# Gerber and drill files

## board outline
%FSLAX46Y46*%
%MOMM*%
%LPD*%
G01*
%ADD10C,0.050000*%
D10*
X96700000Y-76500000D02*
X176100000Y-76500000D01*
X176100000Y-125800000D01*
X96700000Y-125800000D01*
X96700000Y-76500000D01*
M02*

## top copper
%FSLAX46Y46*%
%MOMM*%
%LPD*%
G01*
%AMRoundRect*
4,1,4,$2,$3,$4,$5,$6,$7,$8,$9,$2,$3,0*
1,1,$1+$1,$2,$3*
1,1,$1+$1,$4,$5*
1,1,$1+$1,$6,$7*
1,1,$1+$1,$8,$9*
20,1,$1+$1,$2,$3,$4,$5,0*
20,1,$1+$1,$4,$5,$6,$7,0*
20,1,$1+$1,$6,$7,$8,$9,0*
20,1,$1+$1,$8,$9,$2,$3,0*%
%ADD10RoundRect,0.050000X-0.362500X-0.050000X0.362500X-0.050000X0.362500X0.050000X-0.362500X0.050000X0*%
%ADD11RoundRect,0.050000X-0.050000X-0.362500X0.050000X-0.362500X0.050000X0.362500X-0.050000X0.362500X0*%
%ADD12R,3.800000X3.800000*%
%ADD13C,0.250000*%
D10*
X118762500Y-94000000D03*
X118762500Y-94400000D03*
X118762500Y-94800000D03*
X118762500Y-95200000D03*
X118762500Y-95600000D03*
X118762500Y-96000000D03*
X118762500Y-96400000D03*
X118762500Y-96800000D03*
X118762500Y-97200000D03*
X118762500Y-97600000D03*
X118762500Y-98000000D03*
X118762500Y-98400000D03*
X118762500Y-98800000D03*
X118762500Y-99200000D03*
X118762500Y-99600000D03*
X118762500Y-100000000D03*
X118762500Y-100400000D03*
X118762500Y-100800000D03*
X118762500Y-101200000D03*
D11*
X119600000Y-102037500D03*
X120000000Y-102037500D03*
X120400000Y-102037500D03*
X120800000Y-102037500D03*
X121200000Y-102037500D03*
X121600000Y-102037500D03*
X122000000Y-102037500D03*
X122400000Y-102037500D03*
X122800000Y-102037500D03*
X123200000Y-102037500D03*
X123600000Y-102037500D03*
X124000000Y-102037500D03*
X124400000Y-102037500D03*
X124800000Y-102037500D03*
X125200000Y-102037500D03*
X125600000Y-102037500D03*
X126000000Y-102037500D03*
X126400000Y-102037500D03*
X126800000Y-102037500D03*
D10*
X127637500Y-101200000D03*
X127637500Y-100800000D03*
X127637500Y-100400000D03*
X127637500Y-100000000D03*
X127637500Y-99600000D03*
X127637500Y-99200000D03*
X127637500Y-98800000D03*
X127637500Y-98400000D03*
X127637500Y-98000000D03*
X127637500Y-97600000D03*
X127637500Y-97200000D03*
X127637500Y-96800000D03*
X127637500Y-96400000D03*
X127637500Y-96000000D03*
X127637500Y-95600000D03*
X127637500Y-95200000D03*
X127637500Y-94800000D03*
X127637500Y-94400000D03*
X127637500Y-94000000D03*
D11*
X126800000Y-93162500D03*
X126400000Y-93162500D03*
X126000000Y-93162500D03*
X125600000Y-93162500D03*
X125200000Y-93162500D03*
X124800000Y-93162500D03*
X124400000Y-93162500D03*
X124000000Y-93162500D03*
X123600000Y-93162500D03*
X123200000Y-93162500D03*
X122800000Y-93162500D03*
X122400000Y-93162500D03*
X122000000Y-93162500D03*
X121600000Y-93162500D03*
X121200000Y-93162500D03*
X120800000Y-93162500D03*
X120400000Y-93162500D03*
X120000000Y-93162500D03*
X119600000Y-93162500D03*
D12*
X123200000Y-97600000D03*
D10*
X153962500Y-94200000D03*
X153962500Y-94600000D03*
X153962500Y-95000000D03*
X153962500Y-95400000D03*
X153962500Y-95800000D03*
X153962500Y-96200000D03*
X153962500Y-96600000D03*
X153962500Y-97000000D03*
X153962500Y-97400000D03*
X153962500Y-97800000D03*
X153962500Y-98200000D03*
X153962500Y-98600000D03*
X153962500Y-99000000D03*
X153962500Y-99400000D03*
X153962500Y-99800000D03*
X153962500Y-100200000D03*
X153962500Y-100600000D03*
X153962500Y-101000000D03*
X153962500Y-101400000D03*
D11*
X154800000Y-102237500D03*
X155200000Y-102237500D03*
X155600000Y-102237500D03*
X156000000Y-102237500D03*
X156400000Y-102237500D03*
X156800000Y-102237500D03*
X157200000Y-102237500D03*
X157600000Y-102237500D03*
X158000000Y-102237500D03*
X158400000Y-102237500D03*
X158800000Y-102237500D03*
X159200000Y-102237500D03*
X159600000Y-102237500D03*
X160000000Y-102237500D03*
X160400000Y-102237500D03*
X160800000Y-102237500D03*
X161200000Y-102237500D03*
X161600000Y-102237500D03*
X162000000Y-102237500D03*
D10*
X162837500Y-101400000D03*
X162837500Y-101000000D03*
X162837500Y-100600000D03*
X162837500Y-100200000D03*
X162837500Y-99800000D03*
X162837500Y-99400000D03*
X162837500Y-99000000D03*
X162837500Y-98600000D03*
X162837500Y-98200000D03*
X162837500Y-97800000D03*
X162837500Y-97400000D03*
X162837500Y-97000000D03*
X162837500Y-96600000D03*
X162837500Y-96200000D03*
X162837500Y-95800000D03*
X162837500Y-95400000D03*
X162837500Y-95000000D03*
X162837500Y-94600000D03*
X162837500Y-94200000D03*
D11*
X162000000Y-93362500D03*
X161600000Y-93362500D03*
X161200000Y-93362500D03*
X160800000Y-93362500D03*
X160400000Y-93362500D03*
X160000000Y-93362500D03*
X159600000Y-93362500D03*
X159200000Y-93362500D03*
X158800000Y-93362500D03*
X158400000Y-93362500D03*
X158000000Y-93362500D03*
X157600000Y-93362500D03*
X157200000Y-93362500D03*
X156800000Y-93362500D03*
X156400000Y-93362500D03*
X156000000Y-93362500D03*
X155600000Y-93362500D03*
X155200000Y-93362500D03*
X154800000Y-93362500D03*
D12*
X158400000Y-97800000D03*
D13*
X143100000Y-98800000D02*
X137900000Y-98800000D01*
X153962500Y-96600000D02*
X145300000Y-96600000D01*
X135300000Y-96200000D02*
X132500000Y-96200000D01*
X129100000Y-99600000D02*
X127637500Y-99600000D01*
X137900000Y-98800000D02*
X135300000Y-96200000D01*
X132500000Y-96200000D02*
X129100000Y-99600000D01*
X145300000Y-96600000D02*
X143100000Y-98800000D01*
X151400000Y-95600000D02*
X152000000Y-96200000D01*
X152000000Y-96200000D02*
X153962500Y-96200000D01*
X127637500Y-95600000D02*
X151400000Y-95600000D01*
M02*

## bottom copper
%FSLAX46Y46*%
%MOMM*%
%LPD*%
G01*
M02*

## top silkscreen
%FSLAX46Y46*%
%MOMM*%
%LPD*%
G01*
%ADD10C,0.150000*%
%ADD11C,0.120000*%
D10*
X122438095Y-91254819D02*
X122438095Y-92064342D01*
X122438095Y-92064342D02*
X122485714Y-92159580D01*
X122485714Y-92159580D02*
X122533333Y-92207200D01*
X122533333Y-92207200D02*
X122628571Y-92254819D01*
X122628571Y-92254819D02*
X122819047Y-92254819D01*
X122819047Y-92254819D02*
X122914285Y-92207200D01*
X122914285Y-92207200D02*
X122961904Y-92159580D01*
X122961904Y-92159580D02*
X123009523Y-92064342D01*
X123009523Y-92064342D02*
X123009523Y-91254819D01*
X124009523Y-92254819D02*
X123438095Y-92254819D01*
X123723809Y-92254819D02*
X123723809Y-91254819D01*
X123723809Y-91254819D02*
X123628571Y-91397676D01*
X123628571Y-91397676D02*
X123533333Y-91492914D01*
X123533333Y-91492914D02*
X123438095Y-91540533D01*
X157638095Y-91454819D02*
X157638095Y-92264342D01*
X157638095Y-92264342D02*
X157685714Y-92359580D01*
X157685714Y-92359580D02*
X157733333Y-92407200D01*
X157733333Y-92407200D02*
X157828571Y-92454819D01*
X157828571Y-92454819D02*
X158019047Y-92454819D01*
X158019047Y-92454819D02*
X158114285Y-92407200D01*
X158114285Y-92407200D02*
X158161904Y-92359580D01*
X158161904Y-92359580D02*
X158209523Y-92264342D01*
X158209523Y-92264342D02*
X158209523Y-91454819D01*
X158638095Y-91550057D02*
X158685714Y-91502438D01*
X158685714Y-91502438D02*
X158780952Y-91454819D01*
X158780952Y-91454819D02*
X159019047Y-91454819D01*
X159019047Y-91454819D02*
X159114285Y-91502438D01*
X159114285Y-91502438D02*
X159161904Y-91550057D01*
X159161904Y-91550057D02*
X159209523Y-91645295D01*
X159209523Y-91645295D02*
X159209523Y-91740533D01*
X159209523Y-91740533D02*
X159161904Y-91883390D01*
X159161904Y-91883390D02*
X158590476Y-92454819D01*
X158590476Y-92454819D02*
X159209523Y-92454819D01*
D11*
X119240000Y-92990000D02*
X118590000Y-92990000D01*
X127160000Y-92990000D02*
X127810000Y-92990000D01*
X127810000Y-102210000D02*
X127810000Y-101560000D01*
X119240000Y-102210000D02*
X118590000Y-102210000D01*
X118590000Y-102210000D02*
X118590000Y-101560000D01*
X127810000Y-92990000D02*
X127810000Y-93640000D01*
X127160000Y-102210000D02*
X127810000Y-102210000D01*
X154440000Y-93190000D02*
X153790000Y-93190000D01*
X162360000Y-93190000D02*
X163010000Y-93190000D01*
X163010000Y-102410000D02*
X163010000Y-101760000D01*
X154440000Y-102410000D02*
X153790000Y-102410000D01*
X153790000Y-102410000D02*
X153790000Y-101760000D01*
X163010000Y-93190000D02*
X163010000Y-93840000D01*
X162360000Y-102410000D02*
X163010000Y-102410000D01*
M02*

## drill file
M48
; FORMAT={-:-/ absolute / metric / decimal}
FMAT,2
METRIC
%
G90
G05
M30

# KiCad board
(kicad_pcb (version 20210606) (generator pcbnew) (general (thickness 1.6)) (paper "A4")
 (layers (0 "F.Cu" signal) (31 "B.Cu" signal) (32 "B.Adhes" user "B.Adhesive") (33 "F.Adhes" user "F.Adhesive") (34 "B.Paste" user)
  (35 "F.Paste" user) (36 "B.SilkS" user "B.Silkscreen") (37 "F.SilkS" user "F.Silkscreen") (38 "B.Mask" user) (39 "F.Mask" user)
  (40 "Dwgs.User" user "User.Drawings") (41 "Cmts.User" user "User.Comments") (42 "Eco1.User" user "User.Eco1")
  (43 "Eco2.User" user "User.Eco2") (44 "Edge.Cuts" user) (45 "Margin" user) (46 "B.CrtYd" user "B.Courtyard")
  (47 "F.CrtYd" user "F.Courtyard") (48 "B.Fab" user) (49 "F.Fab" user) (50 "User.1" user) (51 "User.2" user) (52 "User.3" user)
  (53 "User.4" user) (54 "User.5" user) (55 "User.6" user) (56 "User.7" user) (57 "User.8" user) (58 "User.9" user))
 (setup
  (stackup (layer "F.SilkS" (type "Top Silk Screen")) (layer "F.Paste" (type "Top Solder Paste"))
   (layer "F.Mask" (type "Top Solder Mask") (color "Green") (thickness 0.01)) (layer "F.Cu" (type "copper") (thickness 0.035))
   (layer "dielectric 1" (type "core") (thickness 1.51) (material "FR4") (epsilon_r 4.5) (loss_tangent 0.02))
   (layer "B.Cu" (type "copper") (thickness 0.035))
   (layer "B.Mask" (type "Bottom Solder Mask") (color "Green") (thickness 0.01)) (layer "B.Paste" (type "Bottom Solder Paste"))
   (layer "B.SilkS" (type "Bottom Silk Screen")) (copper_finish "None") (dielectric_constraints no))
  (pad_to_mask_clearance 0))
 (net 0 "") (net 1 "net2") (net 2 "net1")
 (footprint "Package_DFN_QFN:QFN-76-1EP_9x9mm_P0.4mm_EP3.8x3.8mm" (layer "F.Cu") (at 123.2 97.6)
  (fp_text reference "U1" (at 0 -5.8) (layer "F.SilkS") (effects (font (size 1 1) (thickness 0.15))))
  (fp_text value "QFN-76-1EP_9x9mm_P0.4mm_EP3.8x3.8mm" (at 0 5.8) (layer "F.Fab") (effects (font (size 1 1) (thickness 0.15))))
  (fp_line (start -3.96 -4.61) (end -4.61 -4.61) (layer "F.SilkS") (width 0.12))
  (fp_line (start 3.96 -4.61) (end 4.61 -4.61) (layer "F.SilkS") (width 0.12))
  (fp_line (start 4.61 4.61) (end 4.61 3.96) (layer "F.SilkS") (width 0.12))
  (fp_line (start -3.96 4.61) (end -4.61 4.61) (layer "F.SilkS") (width 0.12))
  (fp_line (start -4.61 4.61) (end -4.61 3.96) (layer "F.SilkS") (width 0.12))
  (fp_line (start 4.61 -4.61) (end 4.61 -3.96) (layer "F.SilkS") (width 0.12))
  (fp_line (start 3.96 4.61) (end 4.61 4.61) (layer "F.SilkS") (width 0.12))
  (pad "" smd roundrect locked (at 0 -1.27) (size 1.02 1.02) (layers "F.Paste") (roundrect_rratio 0.245098))
  (pad "" smd roundrect locked (at 1.27 -1.27) (size 1.02 1.02) (layers "F.Paste") (roundrect_rratio 0.245098))
  (pad "" smd roundrect locked (at -1.27 -1.27) (size 1.02 1.02) (layers "F.Paste") (roundrect_rratio 0.245098))
  (pad "" smd roundrect locked (at 1.27 1.27) (size 1.02 1.02) (layers "F.Paste") (roundrect_rratio 0.245098))
  (pad "" smd roundrect locked (at 1.27 0) (size 1.02 1.02) (layers "F.Paste") (roundrect_rratio 0.245098))
  (pad "" smd roundrect locked (at -1.27 1.27) (size 1.02 1.02) (layers "F.Paste") (roundrect_rratio 0.245098))
  (pad "" smd roundrect locked (at 0 1.27) (size 1.02 1.02) (layers "F.Paste") (roundrect_rratio 0.245098))
  (pad "" smd roundrect locked (at 0 0) (size 1.02 1.02) (layers "F.Paste") (roundrect_rratio 0.245098))
  (pad "" smd roundrect locked (at -1.27 0) (size 1.02 1.02) (layers "F.Paste") (roundrect_rratio 0.245098))
  (pad "1" smd roundrect locked (at -4.4375 -3.6) (size 0.825 0.2) (layers "F.Cu" "F.Paste" "F.Mask") (roundrect_rratio 0.25))
  (pad "2" smd roundrect locked (at -4.4375 -3.2) (size 0.825 0.2) (layers "F.Cu" "F.Paste" "F.Mask") (roundrect_rratio 0.25))
  (pad "3" smd roundrect locked (at -4.4375 -2.8) (size 0.825 0.2) (layers "F.Cu" "F.Paste" "F.Mask") (roundrect_rratio 0.25))
  (pad "4" smd roundrect locked (at -4.4375 -2.4) (size 0.825 0.2) (layers "F.Cu" "F.Paste" "F.Mask") (roundrect_rratio 0.25))
  (pad "5" smd roundrect locked (at -4.4375 -2) (size 0.825 0.2) (layers "F.Cu" "F.Paste" "F.Mask") (roundrect_rratio 0.25))
  (pad "6" smd roundrect locked (at -4.4375 -1.6) (size 0.825 0.2) (layers "F.Cu" "F.Paste" "F.Mask") (roundrect_rratio 0.25))
  (pad "7" smd roundrect locked (at -4.4375 -1.2) (size 0.825 0.2) (layers "F.Cu" "F.Paste" "F.Mask") (roundrect_rratio 0.25))
  (pad "8" smd roundrect locked (at -4.4375 -0.8) (size 0.825 0.2) (layers "F.Cu" "F.Paste" "F.Mask") (roundrect_rratio 0.25))
  (pad "9" smd roundrect locked (at -4.4375 -0.4) (size 0.825 0.2) (layers "F.Cu" "F.Paste" "F.Mask") (roundrect_rratio 0.25))
  (pad "10" smd roundrect locked (at -4.4375 0) (size 0.825 0.2) (layers "F.Cu" "F.Paste" "F.Mask") (roundrect_rratio 0.25))
  (pad "11" smd roundrect locked (at -4.4375 0.4) (size 0.825 0.2) (layers "F.Cu" "F.Paste" "F.Mask") (roundrect_rratio 0.25))
  (pad "12" smd roundrect locked (at -4.4375 0.8) (size 0.825 0.2) (layers "F.Cu" "F.Paste" "F.Mask") (roundrect_rratio 0.25))
  (pad "13" smd roundrect locked (at -4.4375 1.2) (size 0.825 0.2) (layers "F.Cu" "F.Paste" "F.Mask") (roundrect_rratio 0.25))
  (pad "14" smd roundrect locked (at -4.4375 1.6) (size 0.825 0.2) (layers "F.Cu" "F.Paste" "F.Mask") (roundrect_rratio 0.25))
  (pad "15" smd roundrect locked (at -4.4375 2) (size 0.825 0.2) (layers "F.Cu" "F.Paste" "F.Mask") (roundrect_rratio 0.25))
  (pad "16" smd roundrect locked (at -4.4375 2.4) (size 0.825 0.2) (layers "F.Cu" "F.Paste" "F.Mask") (roundrect_rratio 0.25))
  (pad "17" smd roundrect locked (at -4.4375 2.8) (size 0.825 0.2) (layers "F.Cu" "F.Paste" "F.Mask") (roundrect_rratio 0.25))
  (pad "18" smd roundrect locked (at -4.4375 3.2) (size 0.825 0.2) (layers "F.Cu" "F.Paste" "F.Mask") (roundrect_rratio 0.25))
  (pad "19" smd roundrect locked (at -4.4375 3.6) (size 0.825 0.2) (layers "F.Cu" "F.Paste" "F.Mask") (roundrect_rratio 0.25))
  (pad "20" smd roundrect locked (at -3.6 4.4375) (size 0.2 0.825) (layers "F.Cu" "F.Paste" "F.Mask") (roundrect_rratio 0.25))
  (pad "21" smd roundrect locked (at -3.2 4.4375) (size 0.2 0.825) (layers "F.Cu" "F.Paste" "F.Mask") (roundrect_rratio 0.25))
  (pad "22" smd roundrect locked (at -2.8 4.4375) (size 0.2 0.825) (layers "F.Cu" "F.Paste" "F.Mask") (roundrect_rratio 0.25))
  (pad "23" smd roundrect locked (at -2.4 4.4375) (size 0.2 0.825) (layers "F.Cu" "F.Paste" "F.Mask") (roundrect_rratio 0.25))
  (pad "24" smd roundrect locked (at -2 4.4375) (size 0.2 0.825) (layers "F.Cu" "F.Paste" "F.Mask") (roundrect_rratio 0.25))
  (pad "25" smd roundrect locked (at -1.6 4.4375) (size 0.2 0.825) (layers "F.Cu" "F.Paste" "F.Mask") (roundrect_rratio 0.25))
  (pad "26" smd roundrect locked (at -1.2 4.4375) (size 0.2 0.825) (layers "F.Cu" "F.Paste" "F.Mask") (roundrect_rratio 0.25))
  (pad "27" smd roundrect locked (at -0.8 4.4375) (size 0.2 0.825) (layers "F.Cu" "F.Paste" "F.Mask") (roundrect_rratio 0.25))
  (pad "28" smd roundrect locked (at -0.4 4.4375) (size 0.2 0.825) (layers "F.Cu" "F.Paste" "F.Mask") (roundrect_rratio 0.25))
  (pad "29" smd roundrect locked (at 0 4.4375) (size 0.2 0.825) (layers "F.Cu" "F.Paste" "F.Mask") (roundrect_rratio 0.25))
  (pad "30" smd roundrect locked (at 0.4 4.4375) (size 0.2 0.825) (layers "F.Cu" "F.Paste" "F.Mask") (roundrect_rratio 0.25))
  (pad "31" smd roundrect locked (at 0.8 4.4375) (size 0.2 0.825) (layers "F.Cu" "F.Paste" "F.Mask") (roundrect_rratio 0.25))
  (pad "32" smd roundrect locked (at 1.2 4.4375) (size 0.2 0.825) (layers "F.Cu" "F.Paste" "F.Mask") (roundrect_rratio 0.25))
  (pad "33" smd roundrect locked (at 1.6 4.4375) (size 0.2 0.825) (layers "F.Cu" "F.Paste" "F.Mask") (roundrect_rratio 0.25))
  (pad "34" smd roundrect locked (at 2 4.4375) (size 0.2 0.825) (layers "F.Cu" "F.Paste" "F.Mask") (roundrect_rratio 0.25))
  (pad "35" smd roundrect locked (at 2.4 4.4375) (size 0.2 0.825) (layers "F.Cu" "F.Paste" "F.Mask") (roundrect_rratio 0.25))
  (pad "36" smd roundrect locked (at 2.8 4.4375) (size 0.2 0.825) (layers "F.Cu" "F.Paste" "F.Mask") (roundrect_rratio 0.25))
  (pad "37" smd roundrect locked (at 3.2 4.4375) (size 0.2 0.825) (layers "F.Cu" "F.Paste" "F.Mask") (roundrect_rratio 0.25))
  (pad "38" smd roundrect locked (at 3.6 4.4375) (size 0.2 0.825) (layers "F.Cu" "F.Paste" "F.Mask") (roundrect_rratio 0.25))
  (pad "39" smd roundrect locked (at 4.4375 3.6) (size 0.825 0.2) (layers "F.Cu" "F.Paste" "F.Mask") (roundrect_rratio 0.25))
  (pad "40" smd roundrect locked (at 4.4375 3.2) (size 0.825 0.2) (layers "F.Cu" "F.Paste" "F.Mask") (roundrect_rratio 0.25))
  (pad "41" smd roundrect locked (at 4.4375 2.8) (size 0.825 0.2) (layers "F.Cu" "F.Paste" "F.Mask") (roundrect_rratio 0.25))
  (pad "42" smd roundrect locked (at 4.4375 2.4) (size 0.825 0.2) (layers "F.Cu" "F.Paste" "F.Mask") (roundrect_rratio 0.25))
  (pad "43" smd roundrect locked (at 4.4375 2) (size 0.825 0.2) (layers "F.Cu" "F.Paste" "F.Mask") (roundrect_rratio 0.25) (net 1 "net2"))
  (pad "44" smd roundrect locked (at 4.4375 1.6) (size 0.825 0.2) (layers "F.Cu" "F.Paste" "F.Mask") (roundrect_rratio 0.25))
  (pad "45" smd roundrect locked (at 4.4375 1.2) (size 0.825 0.2) (layers "F.Cu" "F.Paste" "F.Mask") (roundrect_rratio 0.25))
  (pad "46" smd roundrect locked (at 4.4375 0.8) (size 0.825 0.2) (layers "F.Cu" "F.Paste" "F.Mask") (roundrect_rratio 0.25))
  (pad "47" smd roundrect locked (at 4.4375 0.4) (size 0.825 0.2) (layers "F.Cu" "F.Paste" "F.Mask") (roundrect_rratio 0.25))
  (pad "48" smd roundrect locked (at 4.4375 0) (size 0.825 0.2) (layers "F.Cu" "F.Paste" "F.Mask") (roundrect_rratio 0.25))
  (pad "49" smd roundrect locked (at 4.4375 -0.4) (size 0.825 0.2) (layers "F.Cu" "F.Paste" "F.Mask") (roundrect_rratio 0.25))
  (pad "50" smd roundrect locked (at 4.4375 -0.8) (size 0.825 0.2) (layers "F.Cu" "F.Paste" "F.Mask") (roundrect_rratio 0.25))
  (pad "51" smd roundrect locked (at 4.4375 -1.2) (size 0.825 0.2) (layers "F.Cu" "F.Paste" "F.Mask") (roundrect_rratio 0.25))
  (pad "52" smd roundrect locked (at 4.4375 -1.6) (size 0.825 0.2) (layers "F.Cu" "F.Paste" "F.Mask") (roundrect_rratio 0.25))
  (pad "53" smd roundrect locked (at 4.4375 -2) (size 0.825 0.2) (layers "F.Cu" "F.Paste" "F.Mask") (roundrect_rratio 0.25) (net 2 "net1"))
  (pad "54" smd roundrect locked (at 4.4375 -2.4) (size 0.825 0.2) (layers "F.Cu" "F.Paste" "F.Mask") (roundrect_rratio 0.25))
  (pad "55" smd roundrect locked (at 4.4375 -2.8) (size 0.825 0.2) (layers "F.Cu" "F.Paste" "F.Mask") (roundrect_rratio 0.25))
  (pad "56" smd roundrect locked (at 4.4375 -3.2) (size 0.825 0.2) (layers "F.Cu" "F.Paste" "F.Mask") (roundrect_rratio 0.25))
  (pad "57" smd roundrect locked (at 4.4375 -3.6) (size 0.825 0.2) (layers "F.Cu" "F.Paste" "F.Mask") (roundrect_rratio 0.25))
  (pad "58" smd roundrect locked (at 3.6 -4.4375) (size 0.2 0.825) (layers "F.Cu" "F.Paste" "F.Mask") (roundrect_rratio 0.25))
  (pad "59" smd roundrect locked (at 3.2 -4.4375) (size 0.2 0.825) (layers "F.Cu" "F.Paste" "F.Mask") (roundrect_rratio 0.25))
  (pad "60" smd roundrect locked (at 2.8 -4.4375) (size 0.2 0.825) (layers "F.Cu" "F.Paste" "F.Mask") (roundrect_rratio 0.25))
  (pad "61" smd roundrect locked (at 2.4 -4.4375) (size 0.2 0.825) (layers "F.Cu" "F.Paste" "F.Mask") (roundrect_rratio 0.25))
  (pad "62" smd roundrect locked (at 2 -4.4375) (size 0.2 0.825) (layers "F.Cu" "F.Paste" "F.Mask") (roundrect_rratio 0.25))
  (pad "63" smd roundrect locked (at 1.6 -4.4375) (size 0.2 0.825) (layers "F.Cu" "F.Paste" "F.Mask") (roundrect_rratio 0.25))
  (pad "64" smd roundrect locked (at 1.2 -4.4375) (size 0.2 0.825) (layers "F.Cu" "F.Paste" "F.Mask") (roundrect_rratio 0.25))
  (pad "65" smd roundrect locked (at 0.8 -4.4375) (size 0.2 0.825) (layers "F.Cu" "F.Paste" "F.Mask") (roundrect_rratio 0.25))
  (pad "66" smd roundrect locked (at 0.4 -4.4375) (size 0.2 0.825) (layers "F.Cu" "F.Paste" "F.Mask") (roundrect_rratio 0.25))
  (pad "67" smd roundrect locked (at 0 -4.4375) (size 0.2 0.825) (layers "F.Cu" "F.Paste" "F.Mask") (roundrect_rratio 0.25))
  (pad "68" smd roundrect locked (at -0.4 -4.4375) (size 0.2 0.825) (layers "F.Cu" "F.Paste" "F.Mask") (roundrect_rratio 0.25))
  (pad "69" smd roundrect locked (at -0.8 -4.4375) (size 0.2 0.825) (layers "F.Cu" "F.Paste" "F.Mask") (roundrect_rratio 0.25))
  (pad "70" smd roundrect locked (at -1.2 -4.4375) (size 0.2 0.825) (layers "F.Cu" "F.Paste" "F.Mask") (roundrect_rratio 0.25))
  (pad "71" smd roundrect locked (at -1.6 -4.4375) (size 0.2 0.825) (layers "F.Cu" "F.Paste" "F.Mask") (roundrect_rratio 0.25))
  (pad "72" smd roundrect locked (at -2 -4.4375) (size 0.2 0.825) (layers "F.Cu" "F.Paste" "F.Mask") (roundrect_rratio 0.25))
  (pad "73" smd roundrect locked (at -2.4 -4.4375) (size 0.2 0.825) (layers "F.Cu" "F.Paste" "F.Mask") (roundrect_rratio 0.25))
  (pad "74" smd roundrect locked (at -2.8 -4.4375) (size 0.2 0.825) (layers "F.Cu" "F.Paste" "F.Mask") (roundrect_rratio 0.25))
  (pad "75" smd roundrect locked (at -3.2 -4.4375) (size 0.2 0.825) (layers "F.Cu" "F.Paste" "F.Mask") (roundrect_rratio 0.25))
  (pad "76" smd roundrect locked (at -3.6 -4.4375) (size 0.2 0.825) (layers "F.Cu" "F.Paste" "F.Mask") (roundrect_rratio 0.25))
  (pad "77" smd rect locked (at 0 0) (size 3.8 3.8) (layers "F.Cu" "F.Mask")))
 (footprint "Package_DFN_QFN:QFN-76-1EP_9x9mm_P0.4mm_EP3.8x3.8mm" (layer "F.Cu") (at 158.4 97.8)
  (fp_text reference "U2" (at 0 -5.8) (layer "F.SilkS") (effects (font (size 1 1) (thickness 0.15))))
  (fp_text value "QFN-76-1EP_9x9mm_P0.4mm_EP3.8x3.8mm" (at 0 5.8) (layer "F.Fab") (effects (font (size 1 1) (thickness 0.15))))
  (fp_line (start -3.96 -4.61) (end -4.61 -4.61) (layer "F.SilkS") (width 0.12))
  (fp_line (start 3.96 -4.61) (end 4.61 -4.61) (layer "F.SilkS") (width 0.12))
  (fp_line (start 4.61 4.61) (end 4.61 3.96) (layer "F.SilkS") (width 0.12))
  (fp_line (start -3.96 4.61) (end -4.61 4.61) (layer "F.SilkS") (width 0.12))
  (fp_line (start -4.61 4.61) (end -4.61 3.96) (layer "F.SilkS") (width 0.12))
  (fp_line (start 4.61 -4.61) (end 4.61 -3.96) (layer "F.SilkS") (width 0.12))
  (fp_line (start 3.96 4.61) (end 4.61 4.61) (layer "F.SilkS") (width 0.12))
  (pad "" smd roundrect locked (at 0 -1.27) (size 1.02 1.02) (layers "F.Paste") (roundrect_rratio 0.245098))
  (pad "" smd roundrect locked (at 1.27 -1.27) (size 1.02 1.02) (layers "F.Paste") (roundrect_rratio 0.245098))
  (pad "" smd roundrect locked (at -1.27 -1.27) (size 1.02 1.02) (layers "F.Paste") (roundrect_rratio 0.245098))
  (pad "" smd roundrect locked (at 1.27 1.27) (size 1.02 1.02) (layers "F.Paste") (roundrect_rratio 0.245098))
  (pad "" smd roundrect locked (at 1.27 0) (size 1.02 1.02) (layers "F.Paste") (roundrect_rratio 0.245098))
  (pad "" smd roundrect locked (at -1.27 1.27) (size 1.02 1.02) (layers "F.Paste") (roundrect_rratio 0.245098))
  (pad "" smd roundrect locked (at 0 1.27) (size 1.02 1.02) (layers "F.Paste") (roundrect_rratio 0.245098))
  (pad "" smd roundrect locked (at 0 0) (size 1.02 1.02) (layers "F.Paste") (roundrect_rratio 0.245098))
  (pad "" smd roundrect locked (at -1.27 0) (size 1.02 1.02) (layers "F.Paste") (roundrect_rratio 0.245098))
  (pad "1" smd roundrect locked (at -4.4375 -3.6) (size 0.825 0.2) (layers "F.Cu" "F.Paste" "F.Mask") (roundrect_rratio 0.25))
  (pad "2" smd roundrect locked (at -4.4375 -3.2) (size 0.825 0.2) (layers "F.Cu" "F.Paste" "F.Mask") (roundrect_rratio 0.25))
  (pad "3" smd roundrect locked (at -4.4375 -2.8) (size 0.825 0.2) (layers "F.Cu" "F.Paste" "F.Mask") (roundrect_rratio 0.25))
  (pad "4" smd roundrect locked (at -4.4375 -2.4) (size 0.825 0.2) (layers "F.Cu" "F.Paste" "F.Mask") (roundrect_rratio 0.25))
  (pad "5" smd roundrect locked (at -4.4375 -2) (size 0.825 0.2) (layers "F.Cu" "F.Paste" "F.Mask") (roundrect_rratio 0.25))
  (pad "6" smd roundrect locked (at -4.4375 -1.6) (size 0.825 0.2) (layers "F.Cu" "F.Paste" "F.Mask") (roundrect_rratio 0.25) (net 2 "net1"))
  (pad "7" smd roundrect locked (at -4.4375 -1.2) (size 0.825 0.2) (layers "F.Cu" "F.Paste" "F.Mask") (roundrect_rratio 0.25) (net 1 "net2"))
  (pad "8" smd roundrect locked (at -4.4375 -0.8) (size 0.825 0.2) (layers "F.Cu" "F.Paste" "F.Mask") (roundrect_rratio 0.25))
  (pad "9" smd roundrect locked (at -4.4375 -0.4) (size 0.825 0.2) (layers "F.Cu" "F.Paste" "F.Mask") (roundrect_rratio 0.25))
  (pad "10" smd roundrect locked (at -4.4375 0) (size 0.825 0.2) (layers "F.Cu" "F.Paste" "F.Mask") (roundrect_rratio 0.25))
  (pad "11" smd roundrect locked (at -4.4375 0.4) (size 0.825 0.2) (layers "F.Cu" "F.Paste" "F.Mask") (roundrect_rratio 0.25))
  (pad "12" smd roundrect locked (at -4.4375 0.8) (size 0.825 0.2) (layers "F.Cu" "F.Paste" "F.Mask") (roundrect_rratio 0.25))
  (pad "13" smd roundrect locked (at -4.4375 1.2) (size 0.825 0.2) (layers "F.Cu" "F.Paste" "F.Mask") (roundrect_rratio 0.25))
  (pad "14" smd roundrect locked (at -4.4375 1.6) (size 0.825 0.2) (layers "F.Cu" "F.Paste" "F.Mask") (roundrect_rratio 0.25))
  (pad "15" smd roundrect locked (at -4.4375 2) (size 0.825 0.2) (layers "F.Cu" "F.Paste" "F.Mask") (roundrect_rratio 0.25))
  (pad "16" smd roundrect locked (at -4.4375 2.4) (size 0.825 0.2) (layers "F.Cu" "F.Paste" "F.Mask") (roundrect_rratio 0.25))
  (pad "17" smd roundrect locked (at -4.4375 2.8) (size 0.825 0.2) (layers "F.Cu" "F.Paste" "F.Mask") (roundrect_rratio 0.25))
  (pad "18" smd roundrect locked (at -4.4375 3.2) (size 0.825 0.2) (layers "F.Cu" "F.Paste" "F.Mask") (roundrect_rratio 0.25))
  (pad "19" smd roundrect locked (at -4.4375 3.6) (size 0.825 0.2) (layers "F.Cu" "F.Paste" "F.Mask") (roundrect_rratio 0.25))
  (pad "20" smd roundrect locked (at -3.6 4.4375) (size 0.2 0.825) (layers "F.Cu" "F.Paste" "F.Mask") (roundrect_rratio 0.25))
  (pad "21" smd roundrect locked (at -3.2 4.4375) (size 0.2 0.825) (layers "F.Cu" "F.Paste" "F.Mask") (roundrect_rratio 0.25))
  (pad "22" smd roundrect locked (at -2.8 4.4375) (size 0.2 0.825) (layers "F.Cu" "F.Paste" "F.Mask") (roundrect_rratio 0.25))
  (pad "23" smd roundrect locked (at -2.4 4.4375) (size 0.2 0.825) (layers "F.Cu" "F.Paste" "F.Mask") (roundrect_rratio 0.25))
  (pad "24" smd roundrect locked (at -2 4.4375) (size 0.2 0.825) (layers "F.Cu" "F.Paste" "F.Mask") (roundrect_rratio 0.25))
  (pad "25" smd roundrect locked (at -1.6 4.4375) (size 0.2 0.825) (layers "F.Cu" "F.Paste" "F.Mask") (roundrect_rratio 0.25))
  (pad "26" smd roundrect locked (at -1.2 4.4375) (size 0.2 0.825) (layers "F.Cu" "F.Paste" "F.Mask") (roundrect_rratio 0.25))
  (pad "27" smd roundrect locked (at -0.8 4.4375) (size 0.2 0.825) (layers "F.Cu" "F.Paste" "F.Mask") (roundrect_rratio 0.25))
  (pad "28" smd roundrect locked (at -0.4 4.4375) (size 0.2 0.825) (layers "F.Cu" "F.Paste" "F.Mask") (roundrect_rratio 0.25))
  (pad "29" smd roundrect locked (at 0 4.4375) (size 0.2 0.825) (layers "F.Cu" "F.Paste" "F.Mask") (roundrect_rratio 0.25))
  (pad "30" smd roundrect locked (at 0.4 4.4375) (size 0.2 0.825) (layers "F.Cu" "F.Paste" "F.Mask") (roundrect_rratio 0.25))
  (pad "31" smd roundrect locked (at 0.8 4.4375) (size 0.2 0.825) (layers "F.Cu" "F.Paste" "F.Mask") (roundrect_rratio 0.25))
  (pad "32" smd roundrect locked (at 1.2 4.4375) (size 0.2 0.825) (layers "F.Cu" "F.Paste" "F.Mask") (roundrect_rratio 0.25))
  (pad "33" smd roundrect locked (at 1.6 4.4375) (size 0.2 0.825) (layers "F.Cu" "F.Paste" "F.Mask") (roundrect_rratio 0.25))
  (pad "34" smd roundrect locked (at 2 4.4375) (size 0.2 0.825) (layers "F.Cu" "F.Paste" "F.Mask") (roundrect_rratio 0.25))
  (pad "35" smd roundrect locked (at 2.4 4.4375) (size 0.2 0.825) (layers "F.Cu" "F.Paste" "F.Mask") (roundrect_rratio 0.25))
  (pad "36" smd roundrect locked (at 2.8 4.4375) (size 0.2 0.825) (layers "F.Cu" "F.Paste" "F.Mask") (roundrect_rratio 0.25))
  (pad "37" smd roundrect locked (at 3.2 4.4375) (size 0.2 0.825) (layers "F.Cu" "F.Paste" "F.Mask") (roundrect_rratio 0.25))
  (pad "38" smd roundrect locked (at 3.6 4.4375) (size 0.2 0.825) (layers "F.Cu" "F.Paste" "F.Mask") (roundrect_rratio 0.25))
  (pad "39" smd roundrect locked (at 4.4375 3.6) (size 0.825 0.2) (layers "F.Cu" "F.Paste" "F.Mask") (roundrect_rratio 0.25))
  (pad "40" smd roundrect locked (at 4.4375 3.2) (size 0.825 0.2) (layers "F.Cu" "F.Paste" "F.Mask") (roundrect_rratio 0.25))
  (pad "41" smd roundrect locked (at 4.4375 2.8) (size 0.825 0.2) (layers "F.Cu" "F.Paste" "F.Mask") (roundrect_rratio 0.25))
  (pad "42" smd roundrect locked (at 4.4375 2.4) (size 0.825 0.2) (layers "F.Cu" "F.Paste" "F.Mask") (roundrect_rratio 0.25))
  (pad "43" smd roundrect locked (at 4.4375 2) (size 0.825 0.2) (layers "F.Cu" "F.Paste" "F.Mask") (roundrect_rratio 0.25))
  (pad "44" smd roundrect locked (at 4.4375 1.6) (size 0.825 0.2) (layers "F.Cu" "F.Paste" "F.Mask") (roundrect_rratio 0.25))
  (pad "45" smd roundrect locked (at 4.4375 1.2) (size 0.825 0.2) (layers "F.Cu" "F.Paste" "F.Mask") (roundrect_rratio 0.25))
  (pad "46" smd roundrect locked (at 4.4375 0.8) (size 0.825 0.2) (layers "F.Cu" "F.Paste" "F.Mask") (roundrect_rratio 0.25))
  (pad "47" smd roundrect locked (at 4.4375 0.4) (size 0.825 0.2) (layers "F.Cu" "F.Paste" "F.Mask") (roundrect_rratio 0.25))
  (pad "48" smd roundrect locked (at 4.4375 0) (size 0.825 0.2) (layers "F.Cu" "F.Paste" "F.Mask") (roundrect_rratio 0.25))
  (pad "49" smd roundrect locked (at 4.4375 -0.4) (size 0.825 0.2) (layers "F.Cu" "F.Paste" "F.Mask") (roundrect_rratio 0.25))
  (pad "50" smd roundrect locked (at 4.4375 -0.8) (size 0.825 0.2) (layers "F.Cu" "F.Paste" "F.Mask") (roundrect_rratio 0.25))
  (pad "51" smd roundrect locked (at 4.4375 -1.2) (size 0.825 0.2) (layers "F.Cu" "F.Paste" "F.Mask") (roundrect_rratio 0.25))
  (pad "52" smd roundrect locked (at 4.4375 -1.6) (size 0.825 0.2) (layers "F.Cu" "F.Paste" "F.Mask") (roundrect_rratio 0.25))
  (pad "53" smd roundrect locked (at 4.4375 -2) (size 0.825 0.2) (layers "F.Cu" "F.Paste" "F.Mask") (roundrect_rratio 0.25))
  (pad "54" smd roundrect locked (at 4.4375 -2.4) (size 0.825 0.2) (layers "F.Cu" "F.Paste" "F.Mask") (roundrect_rratio 0.25))
  (pad "55" smd roundrect locked (at 4.4375 -2.8) (size 0.825 0.2) (layers "F.Cu" "F.Paste" "F.Mask") (roundrect_rratio 0.25))
  (pad "56" smd roundrect locked (at 4.4375 -3.2) (size 0.825 0.2) (layers "F.Cu" "F.Paste" "F.Mask") (roundrect_rratio 0.25))
  (pad "57" smd roundrect locked (at 4.4375 -3.6) (size 0.825 0.2) (layers "F.Cu" "F.Paste" "F.Mask") (roundrect_rratio 0.25))
  (pad "58" smd roundrect locked (at 3.6 -4.4375) (size 0.2 0.825) (layers "F.Cu" "F.Paste" "F.Mask") (roundrect_rratio 0.25))
  (pad "59" smd roundrect locked (at 3.2 -4.4375) (size 0.2 0.825) (layers "F.Cu" "F.Paste" "F.Mask") (roundrect_rratio 0.25))
  (pad "60" smd roundrect locked (at 2.8 -4.4375) (size 0.2 0.825) (layers "F.Cu" "F.Paste" "F.Mask") (roundrect_rratio 0.25))
  (pad "61" smd roundrect locked (at 2.4 -4.4375) (size 0.2 0.825) (layers "F.Cu" "F.Paste" "F.Mask") (roundrect_rratio 0.25))
  (pad "62" smd roundrect locked (at 2 -4.4375) (size 0.2 0.825) (layers "F.Cu" "F.Paste" "F.Mask") (roundrect_rratio 0.25))
  (pad "63" smd roundrect locked (at 1.6 -4.4375) (size 0.2 0.825) (layers "F.Cu" "F.Paste" "F.Mask") (roundrect_rratio 0.25))
  (pad "64" smd roundrect locked (at 1.2 -4.4375) (size 0.2 0.825) (layers "F.Cu" "F.Paste" "F.Mask") (roundrect_rratio 0.25))
  (pad "65" smd roundrect locked (at 0.8 -4.4375) (size 0.2 0.825) (layers "F.Cu" "F.Paste" "F.Mask") (roundrect_rratio 0.25))
  (pad "66" smd roundrect locked (at 0.4 -4.4375) (size 0.2 0.825) (layers "F.Cu" "F.Paste" "F.Mask") (roundrect_rratio 0.25))
  (pad "67" smd roundrect locked (at 0 -4.4375) (size 0.2 0.825) (layers "F.Cu" "F.Paste" "F.Mask") (roundrect_rratio 0.25))
  (pad "68" smd roundrect locked (at -0.4 -4.4375) (size 0.2 0.825) (layers "F.Cu" "F.Paste" "F.Mask") (roundrect_rratio 0.25))
  (pad "69" smd roundrect locked (at -0.8 -4.4375) (size 0.2 0.825) (layers "F.Cu" "F.Paste" "F.Mask") (roundrect_rratio 0.25))
  (pad "70" smd roundrect locked (at -1.2 -4.4375) (size 0.2 0.825) (layers "F.Cu" "F.Paste" "F.Mask") (roundrect_rratio 0.25))
  (pad "71" smd roundrect locked (at -1.6 -4.4375) (size 0.2 0.825) (layers "F.Cu" "F.Paste" "F.Mask") (roundrect_rratio 0.25))
  (pad "72" smd roundrect locked (at -2 -4.4375) (size 0.2 0.825) (layers "F.Cu" "F.Paste" "F.Mask") (roundrect_rratio 0.25))
  (pad "73" smd roundrect locked (at -2.4 -4.4375) (size 0.2 0.825) (layers "F.Cu" "F.Paste" "F.Mask") (roundrect_rratio 0.25))
  (pad "74" smd roundrect locked (at -2.8 -4.4375) (size 0.2 0.825) (layers "F.Cu" "F.Paste" "F.Mask") (roundrect_rratio 0.25))
  (pad "75" smd roundrect locked (at -3.2 -4.4375) (size 0.2 0.825) (layers "F.Cu" "F.Paste" "F.Mask") (roundrect_rratio 0.25))
  (pad "76" smd roundrect locked (at -3.6 -4.4375) (size 0.2 0.825) (layers "F.Cu" "F.Paste" "F.Mask") (roundrect_rratio 0.25))
  (pad "77" smd rect locked (at 0 0) (size 3.8 3.8) (layers "F.Cu" "F.Mask")))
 (gr_rect (start 96.7 76.5) (end 176.1 125.8) (layer "Edge.Cuts") (width 0.05) (fill none))
 (segment (start 143.1 98.8) (end 137.9 98.8) (width 0.25) (layer "F.Cu") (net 1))
 (segment (start 153.9625 96.6) (end 145.3 96.6) (width 0.25) (layer "F.Cu") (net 1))
 (segment (start 135.3 96.2) (end 132.5 96.2) (width 0.25) (layer "F.Cu") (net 1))
 (segment (start 129.1 99.6) (end 127.6375 99.6) (width 0.25) (layer "F.Cu") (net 1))
 (segment (start 137.9 98.8) (end 135.3 96.2) (width 0.25) (layer "F.Cu") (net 1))
 (segment (start 132.5 96.2) (end 129.1 99.6) (width 0.25) (layer "F.Cu") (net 1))
 (segment (start 145.3 96.6) (end 143.1 98.8) (width 0.25) (layer "F.Cu") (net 1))
 (segment (start 151.4 95.6) (end 152 96.2) (width 0.25) (layer "F.Cu") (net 2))
 (segment (start 152 96.2) (end 153.9625 96.2) (width 0.25) (layer "F.Cu") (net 2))
 (segment (start 127.6375 95.6) (end 151.4 95.6) (width 0.25) (layer "F.Cu") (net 2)))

